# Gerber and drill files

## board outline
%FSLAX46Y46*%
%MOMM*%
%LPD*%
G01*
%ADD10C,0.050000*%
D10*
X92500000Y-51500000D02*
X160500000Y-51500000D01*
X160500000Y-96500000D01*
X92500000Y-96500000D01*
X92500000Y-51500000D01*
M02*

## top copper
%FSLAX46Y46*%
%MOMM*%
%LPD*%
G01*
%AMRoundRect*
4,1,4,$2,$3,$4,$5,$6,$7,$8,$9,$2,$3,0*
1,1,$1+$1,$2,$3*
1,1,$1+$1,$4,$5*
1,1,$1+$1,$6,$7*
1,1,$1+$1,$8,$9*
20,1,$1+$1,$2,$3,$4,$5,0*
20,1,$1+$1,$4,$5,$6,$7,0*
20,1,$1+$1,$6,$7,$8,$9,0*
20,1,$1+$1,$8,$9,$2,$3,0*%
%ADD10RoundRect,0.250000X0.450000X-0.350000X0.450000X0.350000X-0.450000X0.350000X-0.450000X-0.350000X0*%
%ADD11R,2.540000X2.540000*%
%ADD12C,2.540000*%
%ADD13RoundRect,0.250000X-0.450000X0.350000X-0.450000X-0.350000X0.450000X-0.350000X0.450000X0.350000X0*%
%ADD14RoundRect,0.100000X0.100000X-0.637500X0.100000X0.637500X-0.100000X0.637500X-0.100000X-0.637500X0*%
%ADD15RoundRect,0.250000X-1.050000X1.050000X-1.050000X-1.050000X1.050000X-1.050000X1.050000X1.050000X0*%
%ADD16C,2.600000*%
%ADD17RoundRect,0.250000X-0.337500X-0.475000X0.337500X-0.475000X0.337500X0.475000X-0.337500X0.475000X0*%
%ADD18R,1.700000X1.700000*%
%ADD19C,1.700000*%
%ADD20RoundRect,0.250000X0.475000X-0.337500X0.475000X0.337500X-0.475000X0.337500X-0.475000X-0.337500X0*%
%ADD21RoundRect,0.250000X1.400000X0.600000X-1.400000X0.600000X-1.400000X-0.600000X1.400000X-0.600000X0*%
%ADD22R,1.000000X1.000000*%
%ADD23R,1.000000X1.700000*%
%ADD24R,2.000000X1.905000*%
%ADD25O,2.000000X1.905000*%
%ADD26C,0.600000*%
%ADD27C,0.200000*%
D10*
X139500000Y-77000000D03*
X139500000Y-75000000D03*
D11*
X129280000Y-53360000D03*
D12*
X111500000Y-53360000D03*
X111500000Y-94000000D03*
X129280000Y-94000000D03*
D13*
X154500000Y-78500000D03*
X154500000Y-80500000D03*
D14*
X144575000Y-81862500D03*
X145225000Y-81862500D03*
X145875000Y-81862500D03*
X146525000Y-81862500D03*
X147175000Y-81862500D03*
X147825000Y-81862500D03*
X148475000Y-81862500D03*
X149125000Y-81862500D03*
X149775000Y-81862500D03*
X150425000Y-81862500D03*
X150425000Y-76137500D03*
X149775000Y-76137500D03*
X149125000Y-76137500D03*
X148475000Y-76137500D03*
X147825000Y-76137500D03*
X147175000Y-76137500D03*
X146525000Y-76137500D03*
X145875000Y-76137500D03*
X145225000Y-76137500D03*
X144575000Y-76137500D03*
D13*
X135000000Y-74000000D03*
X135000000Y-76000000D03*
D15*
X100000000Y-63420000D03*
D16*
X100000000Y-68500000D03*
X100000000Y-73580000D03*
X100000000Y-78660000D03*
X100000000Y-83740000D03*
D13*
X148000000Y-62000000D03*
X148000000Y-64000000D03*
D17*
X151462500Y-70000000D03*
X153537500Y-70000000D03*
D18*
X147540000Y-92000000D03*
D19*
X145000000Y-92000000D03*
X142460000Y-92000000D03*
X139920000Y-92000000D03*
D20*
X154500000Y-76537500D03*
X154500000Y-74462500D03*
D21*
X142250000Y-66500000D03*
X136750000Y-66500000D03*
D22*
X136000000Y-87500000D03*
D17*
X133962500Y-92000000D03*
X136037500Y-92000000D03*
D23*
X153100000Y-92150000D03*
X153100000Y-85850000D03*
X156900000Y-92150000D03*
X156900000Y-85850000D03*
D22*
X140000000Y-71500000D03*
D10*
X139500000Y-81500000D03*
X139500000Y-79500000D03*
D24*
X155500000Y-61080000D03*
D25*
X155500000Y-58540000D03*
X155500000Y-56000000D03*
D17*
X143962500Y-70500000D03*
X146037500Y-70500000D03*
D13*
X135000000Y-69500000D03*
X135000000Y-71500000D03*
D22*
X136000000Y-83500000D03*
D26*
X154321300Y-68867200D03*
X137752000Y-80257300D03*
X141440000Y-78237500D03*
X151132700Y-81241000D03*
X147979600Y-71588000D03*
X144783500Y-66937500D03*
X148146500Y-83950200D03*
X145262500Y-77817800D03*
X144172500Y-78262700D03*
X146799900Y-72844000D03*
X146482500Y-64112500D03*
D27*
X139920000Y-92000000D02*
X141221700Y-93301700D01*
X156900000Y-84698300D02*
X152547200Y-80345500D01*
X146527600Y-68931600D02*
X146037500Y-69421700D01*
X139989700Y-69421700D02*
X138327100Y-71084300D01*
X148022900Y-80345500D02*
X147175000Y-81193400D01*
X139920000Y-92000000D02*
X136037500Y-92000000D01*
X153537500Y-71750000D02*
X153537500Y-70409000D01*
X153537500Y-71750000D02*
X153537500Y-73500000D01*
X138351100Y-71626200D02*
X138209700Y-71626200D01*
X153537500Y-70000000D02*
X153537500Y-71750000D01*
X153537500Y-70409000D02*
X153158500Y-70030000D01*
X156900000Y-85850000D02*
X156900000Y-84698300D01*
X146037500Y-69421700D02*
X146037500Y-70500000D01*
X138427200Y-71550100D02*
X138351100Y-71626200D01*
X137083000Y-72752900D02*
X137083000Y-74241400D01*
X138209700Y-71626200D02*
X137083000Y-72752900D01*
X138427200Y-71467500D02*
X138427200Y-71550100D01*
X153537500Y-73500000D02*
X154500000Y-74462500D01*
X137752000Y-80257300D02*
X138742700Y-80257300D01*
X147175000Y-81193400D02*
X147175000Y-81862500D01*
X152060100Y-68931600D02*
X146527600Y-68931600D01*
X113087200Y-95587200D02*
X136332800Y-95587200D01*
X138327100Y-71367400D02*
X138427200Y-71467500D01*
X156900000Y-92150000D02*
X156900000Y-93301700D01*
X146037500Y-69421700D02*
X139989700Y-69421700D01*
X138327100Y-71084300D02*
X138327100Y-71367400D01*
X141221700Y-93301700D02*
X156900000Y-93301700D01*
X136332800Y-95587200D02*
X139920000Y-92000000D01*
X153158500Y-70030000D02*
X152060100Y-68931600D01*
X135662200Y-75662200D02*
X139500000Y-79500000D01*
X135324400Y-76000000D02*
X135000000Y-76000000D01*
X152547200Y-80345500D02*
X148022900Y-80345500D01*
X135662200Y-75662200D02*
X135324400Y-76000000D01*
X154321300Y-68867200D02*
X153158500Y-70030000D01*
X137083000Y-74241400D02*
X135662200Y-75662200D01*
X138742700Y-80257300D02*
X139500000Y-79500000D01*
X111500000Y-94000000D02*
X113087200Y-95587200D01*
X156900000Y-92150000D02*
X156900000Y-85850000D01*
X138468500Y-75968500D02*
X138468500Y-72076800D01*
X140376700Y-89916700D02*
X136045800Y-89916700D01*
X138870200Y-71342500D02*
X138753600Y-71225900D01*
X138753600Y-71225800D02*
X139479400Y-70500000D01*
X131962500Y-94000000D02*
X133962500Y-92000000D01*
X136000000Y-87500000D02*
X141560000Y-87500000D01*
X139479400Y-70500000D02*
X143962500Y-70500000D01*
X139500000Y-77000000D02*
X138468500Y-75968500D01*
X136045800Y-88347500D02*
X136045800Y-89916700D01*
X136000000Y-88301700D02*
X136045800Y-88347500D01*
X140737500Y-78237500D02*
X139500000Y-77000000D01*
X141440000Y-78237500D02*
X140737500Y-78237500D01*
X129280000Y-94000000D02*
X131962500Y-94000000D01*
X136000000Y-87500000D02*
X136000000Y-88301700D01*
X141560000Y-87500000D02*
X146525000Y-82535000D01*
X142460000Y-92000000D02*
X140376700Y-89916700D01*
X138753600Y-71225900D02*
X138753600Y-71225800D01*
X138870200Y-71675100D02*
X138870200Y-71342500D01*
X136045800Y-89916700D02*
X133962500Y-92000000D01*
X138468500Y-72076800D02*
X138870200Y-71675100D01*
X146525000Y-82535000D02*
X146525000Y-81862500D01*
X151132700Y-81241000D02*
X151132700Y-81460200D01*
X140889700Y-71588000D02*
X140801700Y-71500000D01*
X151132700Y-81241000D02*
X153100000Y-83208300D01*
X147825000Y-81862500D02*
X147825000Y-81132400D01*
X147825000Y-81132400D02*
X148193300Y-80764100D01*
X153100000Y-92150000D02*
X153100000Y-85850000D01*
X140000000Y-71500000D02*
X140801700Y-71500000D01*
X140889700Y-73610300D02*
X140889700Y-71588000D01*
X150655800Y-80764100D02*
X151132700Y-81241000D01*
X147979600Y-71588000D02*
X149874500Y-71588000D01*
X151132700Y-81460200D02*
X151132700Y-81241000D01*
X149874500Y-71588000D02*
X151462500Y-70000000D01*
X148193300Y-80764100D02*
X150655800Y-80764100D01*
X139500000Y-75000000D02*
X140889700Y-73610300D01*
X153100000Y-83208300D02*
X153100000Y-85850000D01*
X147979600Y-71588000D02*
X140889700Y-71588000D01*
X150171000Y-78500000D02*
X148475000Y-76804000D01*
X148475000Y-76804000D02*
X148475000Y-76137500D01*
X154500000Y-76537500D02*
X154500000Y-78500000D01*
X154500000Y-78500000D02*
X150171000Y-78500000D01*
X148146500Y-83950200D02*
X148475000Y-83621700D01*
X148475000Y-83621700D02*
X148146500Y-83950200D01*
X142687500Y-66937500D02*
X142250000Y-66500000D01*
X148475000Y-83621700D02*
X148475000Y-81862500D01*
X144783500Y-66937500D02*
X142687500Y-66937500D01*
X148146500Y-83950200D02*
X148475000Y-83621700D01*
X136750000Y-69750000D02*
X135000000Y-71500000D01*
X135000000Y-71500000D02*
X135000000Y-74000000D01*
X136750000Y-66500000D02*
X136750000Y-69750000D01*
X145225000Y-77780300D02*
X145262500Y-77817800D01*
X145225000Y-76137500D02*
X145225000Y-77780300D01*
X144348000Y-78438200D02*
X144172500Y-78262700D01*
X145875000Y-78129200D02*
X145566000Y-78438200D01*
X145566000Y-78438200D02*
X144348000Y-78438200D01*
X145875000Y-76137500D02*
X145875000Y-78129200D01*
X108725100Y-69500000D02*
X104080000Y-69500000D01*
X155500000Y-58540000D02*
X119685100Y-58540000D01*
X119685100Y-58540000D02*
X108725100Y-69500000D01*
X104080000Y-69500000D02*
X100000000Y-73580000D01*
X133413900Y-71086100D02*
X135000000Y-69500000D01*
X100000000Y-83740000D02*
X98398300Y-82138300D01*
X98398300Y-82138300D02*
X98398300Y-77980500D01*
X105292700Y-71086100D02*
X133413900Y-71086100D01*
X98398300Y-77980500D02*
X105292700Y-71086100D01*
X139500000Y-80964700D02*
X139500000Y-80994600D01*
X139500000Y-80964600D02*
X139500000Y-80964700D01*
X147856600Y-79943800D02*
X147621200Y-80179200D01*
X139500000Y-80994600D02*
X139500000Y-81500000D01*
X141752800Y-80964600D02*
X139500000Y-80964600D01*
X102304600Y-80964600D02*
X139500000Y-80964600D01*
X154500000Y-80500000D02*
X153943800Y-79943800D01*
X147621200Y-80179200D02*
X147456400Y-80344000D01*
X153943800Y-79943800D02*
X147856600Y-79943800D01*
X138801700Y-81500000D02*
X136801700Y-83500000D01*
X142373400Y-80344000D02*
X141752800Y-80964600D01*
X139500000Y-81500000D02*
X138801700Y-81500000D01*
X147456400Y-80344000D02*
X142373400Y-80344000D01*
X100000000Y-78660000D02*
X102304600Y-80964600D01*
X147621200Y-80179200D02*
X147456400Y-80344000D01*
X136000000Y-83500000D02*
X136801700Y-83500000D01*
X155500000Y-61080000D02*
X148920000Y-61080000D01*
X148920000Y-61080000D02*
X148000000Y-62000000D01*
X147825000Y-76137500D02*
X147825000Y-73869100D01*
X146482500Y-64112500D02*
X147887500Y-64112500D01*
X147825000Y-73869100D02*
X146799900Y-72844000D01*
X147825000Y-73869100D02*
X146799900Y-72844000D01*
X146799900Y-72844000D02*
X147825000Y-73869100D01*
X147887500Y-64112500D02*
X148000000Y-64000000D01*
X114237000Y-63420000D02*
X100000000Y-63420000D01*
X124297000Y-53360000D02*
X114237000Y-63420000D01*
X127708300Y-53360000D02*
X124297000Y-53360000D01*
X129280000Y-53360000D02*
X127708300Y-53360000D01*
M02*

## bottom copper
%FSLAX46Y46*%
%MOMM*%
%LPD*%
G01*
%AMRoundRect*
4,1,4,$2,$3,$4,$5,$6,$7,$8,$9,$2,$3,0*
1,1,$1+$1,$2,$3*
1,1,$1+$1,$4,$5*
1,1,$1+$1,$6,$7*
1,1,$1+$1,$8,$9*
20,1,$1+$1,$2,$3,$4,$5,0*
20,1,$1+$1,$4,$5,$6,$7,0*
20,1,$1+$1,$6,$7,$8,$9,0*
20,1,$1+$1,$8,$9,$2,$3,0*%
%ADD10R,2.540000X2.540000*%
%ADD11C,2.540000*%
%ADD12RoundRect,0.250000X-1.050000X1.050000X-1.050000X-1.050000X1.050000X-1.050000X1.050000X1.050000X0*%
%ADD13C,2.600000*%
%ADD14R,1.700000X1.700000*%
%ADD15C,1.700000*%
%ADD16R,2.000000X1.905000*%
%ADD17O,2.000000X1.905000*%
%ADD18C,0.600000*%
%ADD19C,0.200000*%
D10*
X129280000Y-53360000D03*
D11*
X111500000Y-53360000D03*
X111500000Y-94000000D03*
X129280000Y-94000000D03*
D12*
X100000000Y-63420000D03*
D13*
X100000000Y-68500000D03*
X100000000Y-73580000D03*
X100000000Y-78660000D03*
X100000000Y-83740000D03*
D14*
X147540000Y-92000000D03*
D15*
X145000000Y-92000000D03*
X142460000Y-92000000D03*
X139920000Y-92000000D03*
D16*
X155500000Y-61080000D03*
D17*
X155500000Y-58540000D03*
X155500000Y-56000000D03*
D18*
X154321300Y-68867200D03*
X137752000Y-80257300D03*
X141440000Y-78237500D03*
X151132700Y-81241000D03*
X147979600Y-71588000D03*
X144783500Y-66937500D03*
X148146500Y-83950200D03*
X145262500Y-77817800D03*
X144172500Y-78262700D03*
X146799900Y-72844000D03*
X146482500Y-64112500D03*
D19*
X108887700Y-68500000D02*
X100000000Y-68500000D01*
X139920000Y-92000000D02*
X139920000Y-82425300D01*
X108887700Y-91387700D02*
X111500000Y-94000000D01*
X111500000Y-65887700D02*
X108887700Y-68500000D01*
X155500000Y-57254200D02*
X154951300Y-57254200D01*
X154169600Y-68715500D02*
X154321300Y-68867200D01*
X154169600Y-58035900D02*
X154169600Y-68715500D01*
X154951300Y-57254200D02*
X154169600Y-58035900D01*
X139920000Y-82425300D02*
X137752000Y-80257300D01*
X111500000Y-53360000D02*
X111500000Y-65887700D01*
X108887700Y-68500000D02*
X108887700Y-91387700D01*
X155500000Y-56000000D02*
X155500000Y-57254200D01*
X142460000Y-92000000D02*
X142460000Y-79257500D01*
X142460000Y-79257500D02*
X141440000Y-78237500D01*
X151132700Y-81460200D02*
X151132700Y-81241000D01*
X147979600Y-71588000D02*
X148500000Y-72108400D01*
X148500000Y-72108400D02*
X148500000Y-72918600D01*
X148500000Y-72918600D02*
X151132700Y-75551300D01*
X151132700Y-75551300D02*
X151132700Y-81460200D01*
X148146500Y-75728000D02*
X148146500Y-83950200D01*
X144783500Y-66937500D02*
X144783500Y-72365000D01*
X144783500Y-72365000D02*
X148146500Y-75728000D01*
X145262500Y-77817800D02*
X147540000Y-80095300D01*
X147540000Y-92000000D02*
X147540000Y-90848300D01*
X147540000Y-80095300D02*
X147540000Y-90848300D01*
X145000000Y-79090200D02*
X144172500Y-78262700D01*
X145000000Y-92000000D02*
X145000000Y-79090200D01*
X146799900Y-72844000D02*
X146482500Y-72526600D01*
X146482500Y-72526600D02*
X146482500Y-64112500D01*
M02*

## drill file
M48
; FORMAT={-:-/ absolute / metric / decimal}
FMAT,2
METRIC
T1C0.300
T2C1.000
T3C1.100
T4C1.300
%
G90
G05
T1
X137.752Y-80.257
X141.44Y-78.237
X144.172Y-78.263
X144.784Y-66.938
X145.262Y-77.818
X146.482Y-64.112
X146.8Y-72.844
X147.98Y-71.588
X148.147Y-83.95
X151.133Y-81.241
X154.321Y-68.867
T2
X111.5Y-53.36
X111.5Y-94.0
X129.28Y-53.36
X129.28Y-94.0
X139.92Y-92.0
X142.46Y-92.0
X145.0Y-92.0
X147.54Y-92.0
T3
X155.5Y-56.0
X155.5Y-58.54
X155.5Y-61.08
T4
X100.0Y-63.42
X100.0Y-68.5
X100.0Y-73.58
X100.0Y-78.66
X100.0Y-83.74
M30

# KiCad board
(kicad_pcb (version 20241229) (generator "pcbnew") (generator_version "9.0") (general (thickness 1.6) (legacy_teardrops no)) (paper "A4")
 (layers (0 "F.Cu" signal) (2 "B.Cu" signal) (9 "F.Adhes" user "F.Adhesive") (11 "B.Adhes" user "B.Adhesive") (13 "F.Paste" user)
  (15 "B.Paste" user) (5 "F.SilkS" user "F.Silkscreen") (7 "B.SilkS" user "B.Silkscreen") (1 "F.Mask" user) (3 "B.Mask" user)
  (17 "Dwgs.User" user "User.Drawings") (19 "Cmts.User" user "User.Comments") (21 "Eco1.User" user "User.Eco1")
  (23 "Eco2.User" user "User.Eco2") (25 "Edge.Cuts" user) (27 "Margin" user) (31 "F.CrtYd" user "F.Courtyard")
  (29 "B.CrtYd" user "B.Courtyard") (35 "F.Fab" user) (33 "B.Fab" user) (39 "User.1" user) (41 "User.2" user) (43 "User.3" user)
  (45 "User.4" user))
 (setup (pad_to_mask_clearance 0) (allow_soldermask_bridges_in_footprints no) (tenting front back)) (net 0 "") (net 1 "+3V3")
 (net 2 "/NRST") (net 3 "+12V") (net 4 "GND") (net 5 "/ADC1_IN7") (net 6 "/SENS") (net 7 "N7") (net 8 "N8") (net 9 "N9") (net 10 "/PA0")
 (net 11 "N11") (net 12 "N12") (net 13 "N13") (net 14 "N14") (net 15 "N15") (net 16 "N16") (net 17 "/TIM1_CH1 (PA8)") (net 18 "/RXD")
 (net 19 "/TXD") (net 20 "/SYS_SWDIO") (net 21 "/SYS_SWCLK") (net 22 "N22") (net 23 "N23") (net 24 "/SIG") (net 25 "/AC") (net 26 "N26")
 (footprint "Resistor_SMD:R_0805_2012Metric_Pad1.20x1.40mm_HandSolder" (layer "F.Cu") (at 139.5 76 90)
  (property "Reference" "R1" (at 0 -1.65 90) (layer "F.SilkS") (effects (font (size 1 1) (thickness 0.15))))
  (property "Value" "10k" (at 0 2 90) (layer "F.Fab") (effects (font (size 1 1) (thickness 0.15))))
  (pad "1" smd roundrect (at -1 0 90) (size 1.2 1.4) (layers "F.Cu" "F.Mask" "F.Paste") (roundrect_rratio 0.208333) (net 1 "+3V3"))
  (pad "2" smd roundrect (at 1 0 90) (size 1.2 1.4) (layers "F.Cu" "F.Mask" "F.Paste") (roundrect_rratio 0.208333) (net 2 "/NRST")))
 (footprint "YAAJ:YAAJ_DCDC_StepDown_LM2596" (layer "F.Cu") (at 129.28 53.36 -90)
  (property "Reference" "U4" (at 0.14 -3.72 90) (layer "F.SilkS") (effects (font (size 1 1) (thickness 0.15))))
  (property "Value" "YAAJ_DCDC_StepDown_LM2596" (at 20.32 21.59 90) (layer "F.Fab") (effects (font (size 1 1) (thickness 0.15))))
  (pad "1" thru_hole rect (at 0 0 270) (size 2.54 2.54) (drill 1) (layers "*.Cu" "*.Mask") (remove_unused_layers no) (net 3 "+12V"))
  (pad "2" thru_hole circle (at 0 17.78 270) (size 2.54 2.54) (drill 1) (layers "*.Cu" "*.Mask") (remove_unused_layers no) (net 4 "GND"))
  (pad "3" thru_hole circle (at 40.64 17.78 270) (size 2.54 2.54) (drill 1) (layers "*.Cu" "*.Mask") (remove_unused_layers no) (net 4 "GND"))
  (pad "4" thru_hole circle (at 40.64 0 270) (size 2.54 2.54) (drill 1) (layers "*.Cu" "*.Mask") (remove_unused_layers no) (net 1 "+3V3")))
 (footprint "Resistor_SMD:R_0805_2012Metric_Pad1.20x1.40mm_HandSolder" (layer "F.Cu") (at 154.5 79.5 -90)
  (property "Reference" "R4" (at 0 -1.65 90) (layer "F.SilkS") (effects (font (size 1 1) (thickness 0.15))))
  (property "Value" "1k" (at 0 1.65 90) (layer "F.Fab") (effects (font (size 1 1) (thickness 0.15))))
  (pad "1" smd roundrect (at -1 0 270) (size 1.2 1.4) (layers "F.Cu" "F.Mask" "F.Paste") (roundrect_rratio 0.208333) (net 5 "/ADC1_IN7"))
  (pad "2" smd roundrect (at 1 0 270) (size 1.2 1.4) (layers "F.Cu" "F.Mask" "F.Paste") (roundrect_rratio 0.208333) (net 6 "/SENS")))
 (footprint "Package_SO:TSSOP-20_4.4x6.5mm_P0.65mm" (layer "F.Cu") (at 147.5 79 90)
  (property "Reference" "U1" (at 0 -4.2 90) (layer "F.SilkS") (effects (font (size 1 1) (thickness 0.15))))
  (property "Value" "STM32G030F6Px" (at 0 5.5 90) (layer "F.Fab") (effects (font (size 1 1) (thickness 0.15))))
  (pad "1" smd roundrect (at -2.8625 -2.925 90) (size 1.475 0.4) (layers "F.Cu" "F.Mask" "F.Paste") (roundrect_rratio 0.25) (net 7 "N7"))
  (pad "2" smd roundrect (at -2.8625 -2.275 90) (size 1.475 0.4) (layers "F.Cu" "F.Mask" "F.Paste") (roundrect_rratio 0.25) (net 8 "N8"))
  (pad "3" smd roundrect (at -2.8625 -1.625 90) (size 1.475 0.4) (layers "F.Cu" "F.Mask" "F.Paste") (roundrect_rratio 0.25) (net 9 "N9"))
  (pad "4" smd roundrect (at -2.8625 -0.975 90) (size 1.475 0.4) (layers "F.Cu" "F.Mask" "F.Paste") (roundrect_rratio 0.25) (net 1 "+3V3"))
  (pad "5" smd roundrect (at -2.8625 -0.325 90) (size 1.475 0.4) (layers "F.Cu" "F.Mask" "F.Paste") (roundrect_rratio 0.25) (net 4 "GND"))
  (pad "6" smd roundrect (at -2.8625 0.325 90) (size 1.475 0.4) (layers "F.Cu" "F.Mask" "F.Paste") (roundrect_rratio 0.25) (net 2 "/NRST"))
  (pad "7" smd roundrect (at -2.8625 0.975 90) (size 1.475 0.4) (layers "F.Cu" "F.Mask" "F.Paste") (roundrect_rratio 0.25) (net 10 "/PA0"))
  (pad "8" smd roundrect (at -2.8625 1.625 90) (size 1.475 0.4) (layers "F.Cu" "F.Mask" "F.Paste") (roundrect_rratio 0.25) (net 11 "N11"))
  (pad "9" smd roundrect (at -2.8625 2.275 90) (size 1.475 0.4) (layers "F.Cu" "F.Mask" "F.Paste") (roundrect_rratio 0.25) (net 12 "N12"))
  (pad "10" smd roundrect (at -2.8625 2.925 90) (size 1.475 0.4) (layers "F.Cu" "F.Mask" "F.Paste") (roundrect_rratio 0.25) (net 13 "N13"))
  (pad "11" smd roundrect (at 2.8625 2.925 90) (size 1.475 0.4) (layers "F.Cu" "F.Mask" "F.Paste") (roundrect_rratio 0.25) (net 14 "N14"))
  (pad "12" smd roundrect (at 2.8625 2.275 90) (size 1.475 0.4) (layers "F.Cu" "F.Mask" "F.Paste") (roundrect_rratio 0.25) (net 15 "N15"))
  (pad "13" smd roundrect (at 2.8625 1.625 90) (size 1.475 0.4) (layers "F.Cu" "F.Mask" "F.Paste") (roundrect_rratio 0.25) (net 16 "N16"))
  (pad "14" smd roundrect (at 2.8625 0.975 90) (size 1.475 0.4) (layers "F.Cu" "F.Mask" "F.Paste") (roundrect_rratio 0.25)
   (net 5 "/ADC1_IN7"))
  (pad "15" smd roundrect (at 2.8625 0.325 90) (size 1.475 0.4) (layers "F.Cu" "F.Mask" "F.Paste") (roundrect_rratio 0.25)
   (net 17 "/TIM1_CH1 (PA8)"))
  (pad "16" smd roundrect (at 2.8625 -0.325 90) (size 1.475 0.4) (layers "F.Cu" "F.Mask" "F.Paste") (roundrect_rratio 0.25) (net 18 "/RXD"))
  (pad "17" smd roundrect (at 2.8625 -0.975 90) (size 1.475 0.4) (layers "F.Cu" "F.Mask" "F.Paste") (roundrect_rratio 0.25) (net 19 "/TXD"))
  (pad "18" smd roundrect (at 2.8625 -1.625 90) (size 1.475 0.4) (layers "F.Cu" "F.Mask" "F.Paste") (roundrect_rratio 0.25)
   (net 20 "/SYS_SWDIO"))
  (pad "19" smd roundrect (at 2.8625 -2.275 90) (size 1.475 0.4) (layers "F.Cu" "F.Mask" "F.Paste") (roundrect_rratio 0.25)
   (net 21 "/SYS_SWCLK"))
  (pad "20" smd roundrect (at 2.8625 -2.925 90) (size 1.475 0.4) (layers "F.Cu" "F.Mask" "F.Paste") (roundrect_rratio 0.25) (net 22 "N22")))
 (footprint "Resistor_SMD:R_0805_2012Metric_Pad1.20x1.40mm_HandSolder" (layer "F.Cu") (at 135 75 -90)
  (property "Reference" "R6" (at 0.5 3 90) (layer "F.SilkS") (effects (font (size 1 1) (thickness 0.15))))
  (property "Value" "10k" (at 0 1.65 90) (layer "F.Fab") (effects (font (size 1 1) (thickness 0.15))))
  (pad "1" smd roundrect (at -1 0 270) (size 1.2 1.4) (layers "F.Cu" "F.Mask" "F.Paste") (roundrect_rratio 0.208333) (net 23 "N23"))
  (pad "2" smd roundrect (at 1 0 270) (size 1.2 1.4) (layers "F.Cu" "F.Mask" "F.Paste") (roundrect_rratio 0.208333) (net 4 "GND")))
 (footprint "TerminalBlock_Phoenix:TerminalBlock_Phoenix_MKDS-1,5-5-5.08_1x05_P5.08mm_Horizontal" (layer "F.Cu") (at 100 63.42 -90)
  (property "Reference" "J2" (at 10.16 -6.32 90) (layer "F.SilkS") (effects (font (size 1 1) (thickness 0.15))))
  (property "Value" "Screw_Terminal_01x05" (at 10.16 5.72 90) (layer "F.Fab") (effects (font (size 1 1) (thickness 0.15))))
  (pad "1" thru_hole roundrect (at 0 0 270) (size 2.6 2.6) (drill 1.3) (layers "*.Cu" "*.Mask") (remove_unused_layers no)
   (roundrect_rratio 0.096154) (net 3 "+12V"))
  (pad "2" thru_hole circle (at 5.08 0 270) (size 2.6 2.6) (drill 1.3) (layers "*.Cu" "*.Mask") (remove_unused_layers no) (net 4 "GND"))
  (pad "3" thru_hole circle (at 10.16 0 270) (size 2.6 2.6) (drill 1.3) (layers "*.Cu" "*.Mask") (remove_unused_layers no) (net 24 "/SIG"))
  (pad "4" thru_hole circle (at 15.24 0 270) (size 2.6 2.6) (drill 1.3) (layers "*.Cu" "*.Mask") (remove_unused_layers no) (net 6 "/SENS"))
  (pad "5" thru_hole circle (at 20.32 0 270) (size 2.6 2.6) (drill 1.3) (layers "*.Cu" "*.Mask") (remove_unused_layers no) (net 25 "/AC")))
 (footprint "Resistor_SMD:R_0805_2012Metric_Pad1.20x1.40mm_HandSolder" (layer "F.Cu") (at 148 63 -90)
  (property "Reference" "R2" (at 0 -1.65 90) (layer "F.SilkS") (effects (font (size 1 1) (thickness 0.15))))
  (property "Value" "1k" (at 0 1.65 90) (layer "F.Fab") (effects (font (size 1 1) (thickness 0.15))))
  (pad "1" smd roundrect (at -1 0 270) (size 1.2 1.4) (layers "F.Cu" "F.Mask" "F.Paste") (roundrect_rratio 0.208333) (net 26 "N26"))
  (pad "2" smd roundrect (at 1 0 270) (size 1.2 1.4) (layers "F.Cu" "F.Mask" "F.Paste") (roundrect_rratio 0.208333)
   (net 17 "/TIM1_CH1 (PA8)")))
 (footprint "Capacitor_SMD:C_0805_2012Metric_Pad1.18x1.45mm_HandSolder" (layer "F.Cu") (at 152.5 70)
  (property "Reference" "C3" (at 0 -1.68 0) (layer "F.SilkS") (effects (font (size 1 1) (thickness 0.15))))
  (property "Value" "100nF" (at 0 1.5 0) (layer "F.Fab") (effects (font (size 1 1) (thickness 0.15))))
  (pad "1" smd roundrect (at -1.0375 0) (size 1.175 1.45) (layers "F.Cu" "F.Mask" "F.Paste") (roundrect_rratio 0.212766) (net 2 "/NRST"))
  (pad "2" smd roundrect (at 1.0375 0) (size 1.175 1.45) (layers "F.Cu" "F.Mask" "F.Paste") (roundrect_rratio 0.212766) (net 4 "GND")))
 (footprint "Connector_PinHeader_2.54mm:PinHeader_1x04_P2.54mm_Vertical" (layer "F.Cu") (at 147.54 92 -90)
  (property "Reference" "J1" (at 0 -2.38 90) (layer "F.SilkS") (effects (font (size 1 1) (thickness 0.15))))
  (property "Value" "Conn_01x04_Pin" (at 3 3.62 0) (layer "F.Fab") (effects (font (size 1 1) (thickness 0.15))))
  (pad "1" thru_hole rect (at 0 0 270) (size 1.7 1.7) (drill 1) (layers "*.Cu" "*.Mask") (remove_unused_layers no) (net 21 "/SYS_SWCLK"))
  (pad "2" thru_hole circle (at 0 2.54 270) (size 1.7 1.7) (drill 1) (layers "*.Cu" "*.Mask") (remove_unused_layers no)
   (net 20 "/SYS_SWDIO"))
  (pad "3" thru_hole circle (at 0 5.08 270) (size 1.7 1.7) (drill 1) (layers "*.Cu" "*.Mask") (remove_unused_layers no) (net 1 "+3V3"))
  (pad "4" thru_hole circle (at 0 7.62 270) (size 1.7 1.7) (drill 1) (layers "*.Cu" "*.Mask") (remove_unused_layers no) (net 4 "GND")))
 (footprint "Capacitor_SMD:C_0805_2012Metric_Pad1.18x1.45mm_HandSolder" (layer "F.Cu") (at 154.5 75.5 90)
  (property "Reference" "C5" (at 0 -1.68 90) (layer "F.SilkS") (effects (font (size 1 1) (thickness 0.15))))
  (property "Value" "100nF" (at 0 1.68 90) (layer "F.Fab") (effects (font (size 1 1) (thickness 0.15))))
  (pad "1" smd roundrect (at -1.0375 0 90) (size 1.175 1.45) (layers "F.Cu" "F.Mask" "F.Paste") (roundrect_rratio 0.212766)
   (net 5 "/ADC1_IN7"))
  (pad "2" smd roundrect (at 1.0375 0 90) (size 1.175 1.45) (layers "F.Cu" "F.Mask" "F.Paste") (roundrect_rratio 0.212766) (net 4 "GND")))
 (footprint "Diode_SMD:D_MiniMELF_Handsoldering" (layer "F.Cu") (at 139.5 66.5 180)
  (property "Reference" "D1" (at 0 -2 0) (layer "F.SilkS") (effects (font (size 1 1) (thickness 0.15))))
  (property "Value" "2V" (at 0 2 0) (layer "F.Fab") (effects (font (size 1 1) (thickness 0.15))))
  (pad "1" smd roundrect (at -2.75 0 180) (size 3.3 1.7) (layers "F.Cu" "F.Mask" "F.Paste") (roundrect_rratio 0.1470588235) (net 10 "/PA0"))
  (pad "2" smd roundrect (at 2.75 0 180) (size 3.3 1.7) (layers "F.Cu" "F.Mask" "F.Paste") (roundrect_rratio 0.1470588235) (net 23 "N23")))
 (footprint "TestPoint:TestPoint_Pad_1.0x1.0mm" (layer "F.Cu") (at 136 87.5)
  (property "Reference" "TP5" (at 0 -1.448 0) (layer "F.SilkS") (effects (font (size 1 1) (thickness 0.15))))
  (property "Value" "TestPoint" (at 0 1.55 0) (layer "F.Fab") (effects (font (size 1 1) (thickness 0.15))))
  (pad "1" smd rect (at 0 0) (size 1 1) (layers "F.Cu" "F.Mask") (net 1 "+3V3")))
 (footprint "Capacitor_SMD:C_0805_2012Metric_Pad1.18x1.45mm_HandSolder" (layer "F.Cu") (at 135 92)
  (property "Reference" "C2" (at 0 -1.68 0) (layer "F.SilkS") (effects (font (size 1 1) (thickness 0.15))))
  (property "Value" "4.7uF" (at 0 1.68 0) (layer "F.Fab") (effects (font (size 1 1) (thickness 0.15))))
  (pad "1" smd roundrect (at -1.0375 0) (size 1.175 1.45) (layers "F.Cu" "F.Mask" "F.Paste") (roundrect_rratio 0.212766) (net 1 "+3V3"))
  (pad "2" smd roundrect (at 1.0375 0) (size 1.175 1.45) (layers "F.Cu" "F.Mask" "F.Paste") (roundrect_rratio 0.212766) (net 4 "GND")))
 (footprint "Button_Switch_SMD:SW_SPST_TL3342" (layer "F.Cu") (at 155 89 90)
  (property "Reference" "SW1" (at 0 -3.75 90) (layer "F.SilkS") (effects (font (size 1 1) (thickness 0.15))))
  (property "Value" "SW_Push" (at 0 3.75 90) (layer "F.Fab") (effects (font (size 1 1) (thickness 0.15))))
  (pad "1" smd rect (at -3.15 -1.9 90) (size 1.7 1) (layers "F.Cu" "F.Mask" "F.Paste") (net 2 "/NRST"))
  (pad "1" smd rect (at 3.15 -1.9 90) (size 1.7 1) (layers "F.Cu" "F.Mask" "F.Paste") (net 2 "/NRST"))
  (pad "2" smd rect (at -3.15 1.9 90) (size 1.7 1) (layers "F.Cu" "F.Mask" "F.Paste") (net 4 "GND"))
  (pad "2" smd rect (at 3.15 1.9 90) (size 1.7 1) (layers "F.Cu" "F.Mask" "F.Paste") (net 4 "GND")))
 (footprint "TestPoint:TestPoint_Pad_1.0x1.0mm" (layer "F.Cu") (at 140 71.5)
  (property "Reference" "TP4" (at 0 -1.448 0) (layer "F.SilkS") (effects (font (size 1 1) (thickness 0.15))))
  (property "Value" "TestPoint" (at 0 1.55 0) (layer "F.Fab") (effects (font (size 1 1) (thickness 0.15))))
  (pad "1" smd rect (at 0 0) (size 1 1) (layers "F.Cu" "F.Mask") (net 2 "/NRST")))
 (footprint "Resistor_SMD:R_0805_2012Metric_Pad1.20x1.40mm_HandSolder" (layer "F.Cu") (at 139.5 80.5 90)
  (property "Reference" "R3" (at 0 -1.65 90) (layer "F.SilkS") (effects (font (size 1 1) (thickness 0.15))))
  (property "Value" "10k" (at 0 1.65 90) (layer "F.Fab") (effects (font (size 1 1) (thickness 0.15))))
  (pad "1" smd roundrect (at -1 0 90) (size 1.2 1.4) (layers "F.Cu" "F.Mask" "F.Paste") (roundrect_rratio 0.208333) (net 6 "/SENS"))
  (pad "2" smd roundrect (at 1 0 90) (size 1.2 1.4) (layers "F.Cu" "F.Mask" "F.Paste") (roundrect_rratio 0.208333) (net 4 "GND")))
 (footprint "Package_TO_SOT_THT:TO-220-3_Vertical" (layer "F.Cu") (at 155.5 61.08 90)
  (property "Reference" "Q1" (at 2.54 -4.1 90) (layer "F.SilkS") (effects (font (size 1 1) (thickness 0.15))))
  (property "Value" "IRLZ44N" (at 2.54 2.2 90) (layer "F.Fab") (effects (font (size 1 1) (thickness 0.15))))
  (pad "1" thru_hole rect (at 0 0 90) (size 1.905 2) (drill 1.1) (layers "*.Cu" "*.Mask") (remove_unused_layers no) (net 26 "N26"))
  (pad "2" thru_hole oval (at 2.54 0 90) (size 1.905 2) (drill 1.1) (layers "*.Cu" "*.Mask") (remove_unused_layers no) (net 24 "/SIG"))
  (pad "3" thru_hole oval (at 5.08 0 90) (size 1.905 2) (drill 1.1) (layers "*.Cu" "*.Mask") (remove_unused_layers no) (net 4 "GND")))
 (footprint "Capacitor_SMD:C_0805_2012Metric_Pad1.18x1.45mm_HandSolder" (layer "F.Cu") (at 145 70.5)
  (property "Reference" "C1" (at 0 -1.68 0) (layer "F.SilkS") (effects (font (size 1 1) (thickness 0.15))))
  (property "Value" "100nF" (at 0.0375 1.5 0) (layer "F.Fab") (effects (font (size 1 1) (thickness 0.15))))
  (pad "1" smd roundrect (at -1.0375 0) (size 1.175 1.45) (layers "F.Cu" "F.Mask" "F.Paste") (roundrect_rratio 0.212766) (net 1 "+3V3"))
  (pad "2" smd roundrect (at 1.0375 0) (size 1.175 1.45) (layers "F.Cu" "F.Mask" "F.Paste") (roundrect_rratio 0.212766) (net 4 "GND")))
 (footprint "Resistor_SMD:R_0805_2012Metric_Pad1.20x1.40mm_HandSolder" (layer "F.Cu") (at 135 70.5 -90)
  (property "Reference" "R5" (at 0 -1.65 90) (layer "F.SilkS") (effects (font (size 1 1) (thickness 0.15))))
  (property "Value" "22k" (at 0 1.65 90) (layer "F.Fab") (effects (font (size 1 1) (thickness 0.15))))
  (pad "1" smd roundrect (at -1 0 270) (size 1.2 1.4) (layers "F.Cu" "F.Mask" "F.Paste") (roundrect_rratio 0.208333) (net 25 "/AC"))
  (pad "2" smd roundrect (at 1 0 270) (size 1.2 1.4) (layers "F.Cu" "F.Mask" "F.Paste") (roundrect_rratio 0.208333) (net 23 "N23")))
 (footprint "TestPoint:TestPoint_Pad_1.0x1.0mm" (layer "F.Cu") (at 136 83.5)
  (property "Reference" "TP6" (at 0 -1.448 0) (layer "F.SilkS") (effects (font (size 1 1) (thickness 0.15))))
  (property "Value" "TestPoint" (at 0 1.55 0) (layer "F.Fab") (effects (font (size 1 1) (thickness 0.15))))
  (pad "1" smd rect (at 0 0) (size 1 1) (layers "F.Cu" "F.Mask") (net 6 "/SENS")))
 (gr_rect (start 92.5 51.5) (end 160.5 96.5) (stroke (width 0.05) (type default)) (fill no) (layer "Edge.Cuts"))
 (segment (start 139.92 92) (end 141.2217 93.3017) (width 0.2) (layer "F.Cu") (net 4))
 (segment (start 156.9 84.6983) (end 152.5472 80.3455) (width 0.2) (layer "F.Cu") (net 4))
 (segment (start 146.5276 68.9316) (end 146.0375 69.4217) (width 0.2) (layer "F.Cu") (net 4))
 (segment (start 139.9897 69.4217) (end 138.3271 71.0843) (width 0.2) (layer "F.Cu") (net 4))
 (segment (start 148.0229 80.3455) (end 147.175 81.1934) (width 0.2) (layer "F.Cu") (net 4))
 (segment (start 139.92 92) (end 136.0375 92) (width 0.2) (layer "F.Cu") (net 4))
 (segment (start 153.5375 71.75) (end 153.5375 70.409) (width 0.2) (layer "F.Cu") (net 4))
 (segment (start 153.5375 71.75) (end 153.5375 73.5) (width 0.2) (layer "F.Cu") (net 4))
 (segment (start 138.3511 71.6262) (end 138.2097 71.6262) (width 0.2) (layer "F.Cu") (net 4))
 (segment (start 153.5375 70) (end 153.5375 71.75) (width 0.2) (layer "F.Cu") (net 4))
 (segment (start 153.5375 70.409) (end 153.1585 70.03) (width 0.2) (layer "F.Cu") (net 4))
 (segment (start 156.9 85.85) (end 156.9 84.6983) (width 0.2) (layer "F.Cu") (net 4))
 (segment (start 146.0375 69.4217) (end 146.0375 70.5) (width 0.2) (layer "F.Cu") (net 4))
 (segment (start 138.4272 71.5501) (end 138.3511 71.6262) (width 0.2) (layer "F.Cu") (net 4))
 (segment (start 137.083 72.7529) (end 137.083 74.2414) (width 0.2) (layer "F.Cu") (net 4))
 (segment (start 138.2097 71.6262) (end 137.083 72.7529) (width 0.2) (layer "F.Cu") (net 4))
 (segment (start 138.4272 71.4675) (end 138.4272 71.5501) (width 0.2) (layer "F.Cu") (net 4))
 (segment (start 153.5375 73.5) (end 154.5 74.4625) (width 0.2) (layer "F.Cu") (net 4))
 (segment (start 137.752 80.2573) (end 138.7427 80.2573) (width 0.2) (layer "F.Cu") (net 4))
 (segment (start 147.175 81.1934) (end 147.175 81.8625) (width 0.2) (layer "F.Cu") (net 4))
 (segment (start 152.0601 68.9316) (end 146.5276 68.9316) (width 0.2) (layer "F.Cu") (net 4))
 (segment (start 113.0872 95.5872) (end 136.3328 95.5872) (width 0.2) (layer "F.Cu") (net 4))
 (segment (start 138.3271 71.3674) (end 138.4272 71.4675) (width 0.2) (layer "F.Cu") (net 4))
 (segment (start 156.9 92.15) (end 156.9 93.3017) (width 0.2) (layer "F.Cu") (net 4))
 (segment (start 146.0375 69.4217) (end 139.9897 69.4217) (width 0.2) (layer "F.Cu") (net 4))
 (segment (start 138.3271 71.0843) (end 138.3271 71.3674) (width 0.2) (layer "F.Cu") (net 4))
 (segment (start 141.2217 93.3017) (end 156.9 93.3017) (width 0.2) (layer "F.Cu") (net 4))
 (segment (start 136.3328 95.5872) (end 139.92 92) (width 0.2) (layer "F.Cu") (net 4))
 (segment (start 153.1585 70.03) (end 152.0601 68.9316) (width 0.2) (layer "F.Cu") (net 4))
 (segment (start 135.6622 75.6622) (end 139.5 79.5) (width 0.2) (layer "F.Cu") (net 4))
 (segment (start 135.3244 76) (end 135 76) (width 0.2) (layer "F.Cu") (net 4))
 (segment (start 152.5472 80.3455) (end 148.0229 80.3455) (width 0.2) (layer "F.Cu") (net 4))
 (segment (start 135.6622 75.6622) (end 135.3244 76) (width 0.2) (layer "F.Cu") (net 4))
 (segment (start 154.3213 68.8672) (end 153.1585 70.03) (width 0.2) (layer "F.Cu") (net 4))
 (segment (start 137.083 74.2414) (end 135.6622 75.6622) (width 0.2) (layer "F.Cu") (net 4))
 (segment (start 138.7427 80.2573) (end 139.5 79.5) (width 0.2) (layer "F.Cu") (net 4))
 (segment (start 111.5 94) (end 113.0872 95.5872) (width 0.2) (layer "F.Cu") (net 4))
 (segment (start 156.9 92.15) (end 156.9 85.85) (width 0.2) (layer "F.Cu") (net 4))
 (via (at 154.3213 68.8672) (size 0.6) (drill 0.3) (layers "F.Cu" "B.Cu") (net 4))
 (via (at 137.752 80.2573) (size 0.6) (drill 0.3) (layers "F.Cu" "B.Cu") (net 4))
 (segment (start 108.8877 68.5) (end 100 68.5) (width 0.2) (layer "B.Cu") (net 4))
 (segment (start 139.92 92) (end 139.92 82.4253) (width 0.2) (layer "B.Cu") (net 4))
 (segment (start 108.8877 91.3877) (end 111.5 94) (width 0.2) (layer "B.Cu") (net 4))
 (segment (start 111.5 65.8877) (end 108.8877 68.5) (width 0.2) (layer "B.Cu") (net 4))
 (segment (start 155.5 57.2542) (end 154.9513 57.2542) (width 0.2) (layer "B.Cu") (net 4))
 (segment (start 154.1696 68.7155) (end 154.3213 68.8672) (width 0.2) (layer "B.Cu") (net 4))
 (segment (start 154.1696 58.0359) (end 154.1696 68.7155) (width 0.2) (layer "B.Cu") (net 4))
 (segment (start 154.9513 57.2542) (end 154.1696 58.0359) (width 0.2) (layer "B.Cu") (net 4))
 (segment (start 139.92 82.4253) (end 137.752 80.2573) (width 0.2) (layer "B.Cu") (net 4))
 (segment (start 111.5 53.36) (end 111.5 65.8877) (width 0.2) (layer "B.Cu") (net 4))
 (segment (start 108.8877 68.5) (end 108.8877 91.3877) (width 0.2) (layer "B.Cu") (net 4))
 (segment (start 155.5 56) (end 155.5 57.2542) (width 0.2) (layer "B.Cu") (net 4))
 (segment (start 138.4685 75.9685) (end 138.4685 72.0768) (width 0.2) (layer "F.Cu") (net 1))
 (segment (start 140.3767 89.9167) (end 136.0458 89.9167) (width 0.2) (layer "F.Cu") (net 1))
 (segment (start 138.8702 71.3425) (end 138.7536 71.2259) (width 0.2) (layer "F.Cu") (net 1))
 (segment (start 138.7536 71.2258) (end 139.4794 70.5) (width 0.2) (layer "F.Cu") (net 1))
 (segment (start 131.9625 94) (end 133.9625 92) (width 0.2) (layer "F.Cu") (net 1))
 (segment (start 136 87.5) (end 141.56 87.5) (width 0.2) (layer "F.Cu") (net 1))
 (segment (start 139.4794 70.5) (end 143.9625 70.5) (width 0.2) (layer "F.Cu") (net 1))
 (segment (start 139.5 77) (end 138.4685 75.9685) (width 0.2) (layer "F.Cu") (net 1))
 (segment (start 136.0458 88.3475) (end 136.0458 89.9167) (width 0.2) (layer "F.Cu") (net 1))
 (segment (start 136 88.3017) (end 136.0458 88.3475) (width 0.2) (layer "F.Cu") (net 1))
 (segment (start 140.7375 78.2375) (end 139.5 77) (width 0.2) (layer "F.Cu") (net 1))
 (segment (start 141.44 78.2375) (end 140.7375 78.2375) (width 0.2) (layer "F.Cu") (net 1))
 (segment (start 129.28 94) (end 131.9625 94) (width 0.2) (layer "F.Cu") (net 1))
 (segment (start 136 87.5) (end 136 88.3017) (width 0.2) (layer "F.Cu") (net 1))
 (segment (start 141.56 87.5) (end 146.525 82.535) (width 0.2) (layer "F.Cu") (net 1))
 (segment (start 142.46 92) (end 140.3767 89.9167) (width 0.2) (layer "F.Cu") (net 1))
 (segment (start 138.7536 71.2259) (end 138.7536 71.2258) (width 0.2) (layer "F.Cu") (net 1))
 (segment (start 138.8702 71.6751) (end 138.8702 71.3425) (width 0.2) (layer "F.Cu") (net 1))
 (segment (start 136.0458 89.9167) (end 133.9625 92) (width 0.2) (layer "F.Cu") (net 1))
 (segment (start 138.4685 72.0768) (end 138.8702 71.6751) (width 0.2) (layer "F.Cu") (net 1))
 (segment (start 146.525 82.535) (end 146.525 81.8625) (width 0.2) (layer "F.Cu") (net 1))
 (via (at 141.44 78.2375) (size 0.6) (drill 0.3) (layers "F.Cu" "B.Cu") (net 1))
 (segment (start 142.46 92) (end 142.46 79.2575) (width 0.2) (layer "B.Cu") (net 1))
 (segment (start 142.46 79.2575) (end 141.44 78.2375) (width 0.2) (layer "B.Cu") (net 1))
 (segment (start 151.1327 81.241) (end 151.1327 81.4602) (width 0.2) (layer "F.Cu") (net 2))
 (segment (start 140.8897 71.588) (end 140.8017 71.5) (width 0.2) (layer "F.Cu") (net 2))
 (segment (start 151.1327 81.241) (end 153.1 83.2083) (width 0.2) (layer "F.Cu") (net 2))
 (segment (start 147.825 81.8625) (end 147.825 81.1324) (width 0.2) (layer "F.Cu") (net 2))
 (segment (start 147.825 81.1324) (end 148.1933 80.7641) (width 0.2) (layer "F.Cu") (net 2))
 (segment (start 153.1 92.15) (end 153.1 85.85) (width 0.2) (layer "F.Cu") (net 2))
 (segment (start 140 71.5) (end 140.8017 71.5) (width 0.2) (layer "F.Cu") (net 2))
 (segment (start 140.8897 73.6103) (end 140.8897 71.588) (width 0.2) (layer "F.Cu") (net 2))
 (segment (start 150.6558 80.7641) (end 151.1327 81.241) (width 0.2) (layer "F.Cu") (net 2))
 (segment (start 147.9796 71.588) (end 149.8745 71.588) (width 0.2) (layer "F.Cu") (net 2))
 (segment (start 151.1327 81.4602) (end 151.1327 81.241) (width 0.2) (layer "F.Cu") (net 2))
 (segment (start 149.8745 71.588) (end 151.4625 70) (width 0.2) (layer "F.Cu") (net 2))
 (segment (start 148.1933 80.7641) (end 150.6558 80.7641) (width 0.2) (layer "F.Cu") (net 2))
 (segment (start 139.5 75) (end 140.8897 73.6103) (width 0.2) (layer "F.Cu") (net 2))
 (segment (start 153.1 83.2083) (end 153.1 85.85) (width 0.2) (layer "F.Cu") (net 2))
 (segment (start 147.9796 71.588) (end 140.8897 71.588) (width 0.2) (layer "F.Cu") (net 2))
 (via (at 151.1327 81.241) (size 0.6) (drill 0.3) (layers "F.Cu" "B.Cu") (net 2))
 (via (at 147.9796 71.588) (size 0.6) (drill 0.3) (layers "F.Cu" "B.Cu") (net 2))
 (segment (start 151.1327 81.4602) (end 151.1327 81.241) (width 0.2) (layer "B.Cu") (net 2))
 (segment (start 147.9796 71.588) (end 148.5 72.1084) (width 0.2) (layer "B.Cu") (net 2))
 (segment (start 148.5 72.1084) (end 148.5 72.9186) (width 0.2) (layer "B.Cu") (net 2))
 (segment (start 148.5 72.9186) (end 151.1327 75.5513) (width 0.2) (layer "B.Cu") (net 2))
 (segment (start 151.1327 75.5513) (end 151.1327 81.4602) (width 0.2) (layer "B.Cu") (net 2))
 (segment (start 150.171 78.5) (end 148.475 76.804) (width 0.2) (layer "F.Cu") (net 5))
 (segment (start 148.475 76.804) (end 148.475 76.1375) (width 0.2) (layer "F.Cu") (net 5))
 (segment (start 154.5 76.5375) (end 154.5 78.5) (width 0.2) (layer "F.Cu") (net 5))
 (segment (start 154.5 78.5) (end 150.171 78.5) (width 0.2) (layer "F.Cu") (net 5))
 (segment (start 148.1465 83.9502) (end 148.475 83.6217) (width 0.2) (layer "F.Cu") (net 10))
 (segment (start 148.475 83.6217) (end 148.1465 83.9502) (width 0.2) (layer "F.Cu") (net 10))
 (segment (start 142.6875 66.9375) (end 142.25 66.5) (width 0.2) (layer "F.Cu") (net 10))
 (segment (start 148.475 83.6217) (end 148.475 81.8625) (width 0.2) (layer "F.Cu") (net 10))
 (segment (start 144.7835 66.9375) (end 142.6875 66.9375) (width 0.2) (layer "F.Cu") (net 10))
 (segment (start 148.1465 83.9502) (end 148.475 83.6217) (width 0.2) (layer "F.Cu") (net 10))
 (via (at 144.7835 66.9375) (size 0.6) (drill 0.3) (layers "F.Cu" "B.Cu") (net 10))
 (via (at 148.1465 83.9502) (size 0.6) (drill 0.3) (layers "F.Cu" "B.Cu") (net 10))
 (segment (start 148.1465 75.728) (end 148.1465 83.9502) (width 0.2) (layer "B.Cu") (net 10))
 (segment (start 144.7835 66.9375) (end 144.7835 72.365) (width 0.2) (layer "B.Cu") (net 10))
 (segment (start 144.7835 72.365) (end 148.1465 75.728) (width 0.2) (layer "B.Cu") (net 10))
 (segment (start 136.75 69.75) (end 135 71.5) (width 0.2) (layer "F.Cu") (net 23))
 (segment (start 135 71.5) (end 135 74) (width 0.2) (layer "F.Cu") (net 23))
 (segment (start 136.75 66.5) (end 136.75 69.75) (width 0.2) (layer "F.Cu") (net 23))
 (segment (start 145.225 77.7803) (end 145.2625 77.8178) (width 0.2) (layer "F.Cu") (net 21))
 (segment (start 145.225 76.1375) (end 145.225 77.7803) (width 0.2) (layer "F.Cu") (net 21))
 (via (at 145.2625 77.8178) (size 0.6) (drill 0.3) (layers "F.Cu" "B.Cu") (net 21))
 (segment (start 145.2625 77.8178) (end 147.54 80.0953) (width 0.2) (layer "B.Cu") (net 21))
 (segment (start 147.54 92) (end 147.54 90.8483) (width 0.2) (layer "B.Cu") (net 21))
 (segment (start 147.54 80.0953) (end 147.54 90.8483) (width 0.2) (layer "B.Cu") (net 21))
 (segment (start 144.348 78.4382) (end 144.1725 78.2627) (width 0.2) (layer "F.Cu") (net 20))
 (segment (start 145.875 78.1292) (end 145.566 78.4382) (width 0.2) (layer "F.Cu") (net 20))
 (segment (start 145.566 78.4382) (end 144.348 78.4382) (width 0.2) (layer "F.Cu") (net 20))
 (segment (start 145.875 76.1375) (end 145.875 78.1292) (width 0.2) (layer "F.Cu") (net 20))
 (via (at 144.1725 78.2627) (size 0.6) (drill 0.3) (layers "F.Cu" "B.Cu") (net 20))
 (segment (start 145 79.0902) (end 144.1725 78.2627) (width 0.2) (layer "B.Cu") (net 20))
 (segment (start 145 92) (end 145 79.0902) (width 0.2) (layer "B.Cu") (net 20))
 (segment (start 108.7251 69.5) (end 104.08 69.5) (width 0.2) (layer "F.Cu") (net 24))
 (segment (start 155.5 58.54) (end 119.6851 58.54) (width 0.2) (layer "F.Cu") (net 24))
 (segment (start 119.6851 58.54) (end 108.7251 69.5) (width 0.2) (layer "F.Cu") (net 24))
 (segment (start 104.08 69.5) (end 100 73.58) (width 0.2) (layer "F.Cu") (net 24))
 (segment (start 133.4139 71.0861) (end 135 69.5) (width 0.2) (layer "F.Cu") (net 25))
 (segment (start 100 83.74) (end 98.3983 82.1383) (width 0.2) (layer "F.Cu") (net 25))
 (segment (start 98.3983 82.1383) (end 98.3983 77.9805) (width 0.2) (layer "F.Cu") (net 25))
 (segment (start 105.2927 71.0861) (end 133.4139 71.0861) (width 0.2) (layer "F.Cu") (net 25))
 (segment (start 98.3983 77.9805) (end 105.2927 71.0861) (width 0.2) (layer "F.Cu") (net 25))
 (segment (start 139.5 80.9647) (end 139.5 80.9946) (width 0.2) (layer "F.Cu") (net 6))
 (segment (start 139.5 80.9646) (end 139.5 80.9647) (width 0.2) (layer "F.Cu") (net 6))
 (segment (start 147.8566 79.9438) (end 147.6212 80.1792) (width 0.2) (layer "F.Cu") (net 6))
 (segment (start 139.5 80.9946) (end 139.5 81.5) (width 0.2) (layer "F.Cu") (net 6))
 (segment (start 141.7528 80.9646) (end 139.5 80.9646) (width 0.2) (layer "F.Cu") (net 6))
 (segment (start 102.3046 80.9646) (end 139.5 80.9646) (width 0.2) (layer "F.Cu") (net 6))
 (segment (start 154.5 80.5) (end 153.9438 79.9438) (width 0.2) (layer "F.Cu") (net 6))
 (segment (start 147.6212 80.1792) (end 147.4564 80.344) (width 0.2) (layer "F.Cu") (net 6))
 (segment (start 153.9438 79.9438) (end 147.8566 79.9438) (width 0.2) (layer "F.Cu") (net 6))
 (segment (start 138.8017 81.5) (end 136.8017 83.5) (width 0.2) (layer "F.Cu") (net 6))
 (segment (start 142.3734 80.344) (end 141.7528 80.9646) (width 0.2) (layer "F.Cu") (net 6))
 (segment (start 139.5 81.5) (end 138.8017 81.5) (width 0.2) (layer "F.Cu") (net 6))
 (segment (start 147.4564 80.344) (end 142.3734 80.344) (width 0.2) (layer "F.Cu") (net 6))
 (segment (start 100 78.66) (end 102.3046 80.9646) (width 0.2) (layer "F.Cu") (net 6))
 (segment (start 147.6212 80.1792) (end 147.4564 80.344) (width 0.2) (layer "F.Cu") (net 6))
 (segment (start 136 83.5) (end 136.8017 83.5) (width 0.2) (layer "F.Cu") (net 6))
 (segment (start 155.5 61.08) (end 148.92 61.08) (width 0.2) (layer "F.Cu") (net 26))
 (segment (start 148.92 61.08) (end 148 62) (width 0.2) (layer "F.Cu") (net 26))
 (segment (start 147.825 76.1375) (end 147.825 73.8691) (width 0.2) (layer "F.Cu") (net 17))
 (segment (start 146.4825 64.1125) (end 147.8875 64.1125) (width 0.2) (layer "F.Cu") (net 17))
 (segment (start 147.825 73.8691) (end 146.7999 72.844) (width 0.2) (layer "F.Cu") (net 17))
 (segment (start 147.825 73.8691) (end 146.7999 72.844) (width 0.2) (layer "F.Cu") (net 17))
 (segment (start 146.7999 72.844) (end 147.825 73.8691) (width 0.2) (layer "F.Cu") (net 17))
 (segment (start 147.8875 64.1125) (end 148 64) (width 0.2) (layer "F.Cu") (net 17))
 (via (at 146.7999 72.844) (size 0.6) (drill 0.3) (layers "F.Cu" "B.Cu") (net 17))
 (via (at 146.4825 64.1125) (size 0.6) (drill 0.3) (layers "F.Cu" "B.Cu") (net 17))
 (segment (start 146.7999 72.844) (end 146.4825 72.5266) (width 0.2) (layer "B.Cu") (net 17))
 (segment (start 146.4825 72.5266) (end 146.4825 64.1125) (width 0.2) (layer "B.Cu") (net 17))
 (segment (start 114.237 63.42) (end 100 63.42) (width 0.2) (layer "F.Cu") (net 3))
 (segment (start 124.297 53.36) (end 114.237 63.42) (width 0.2) (layer "F.Cu") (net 3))
 (segment (start 127.7083 53.36) (end 124.297 53.36) (width 0.2) (layer "F.Cu") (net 3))
 (segment (start 129.28 53.36) (end 127.7083 53.36) (width 0.2) (layer "F.Cu") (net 3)))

